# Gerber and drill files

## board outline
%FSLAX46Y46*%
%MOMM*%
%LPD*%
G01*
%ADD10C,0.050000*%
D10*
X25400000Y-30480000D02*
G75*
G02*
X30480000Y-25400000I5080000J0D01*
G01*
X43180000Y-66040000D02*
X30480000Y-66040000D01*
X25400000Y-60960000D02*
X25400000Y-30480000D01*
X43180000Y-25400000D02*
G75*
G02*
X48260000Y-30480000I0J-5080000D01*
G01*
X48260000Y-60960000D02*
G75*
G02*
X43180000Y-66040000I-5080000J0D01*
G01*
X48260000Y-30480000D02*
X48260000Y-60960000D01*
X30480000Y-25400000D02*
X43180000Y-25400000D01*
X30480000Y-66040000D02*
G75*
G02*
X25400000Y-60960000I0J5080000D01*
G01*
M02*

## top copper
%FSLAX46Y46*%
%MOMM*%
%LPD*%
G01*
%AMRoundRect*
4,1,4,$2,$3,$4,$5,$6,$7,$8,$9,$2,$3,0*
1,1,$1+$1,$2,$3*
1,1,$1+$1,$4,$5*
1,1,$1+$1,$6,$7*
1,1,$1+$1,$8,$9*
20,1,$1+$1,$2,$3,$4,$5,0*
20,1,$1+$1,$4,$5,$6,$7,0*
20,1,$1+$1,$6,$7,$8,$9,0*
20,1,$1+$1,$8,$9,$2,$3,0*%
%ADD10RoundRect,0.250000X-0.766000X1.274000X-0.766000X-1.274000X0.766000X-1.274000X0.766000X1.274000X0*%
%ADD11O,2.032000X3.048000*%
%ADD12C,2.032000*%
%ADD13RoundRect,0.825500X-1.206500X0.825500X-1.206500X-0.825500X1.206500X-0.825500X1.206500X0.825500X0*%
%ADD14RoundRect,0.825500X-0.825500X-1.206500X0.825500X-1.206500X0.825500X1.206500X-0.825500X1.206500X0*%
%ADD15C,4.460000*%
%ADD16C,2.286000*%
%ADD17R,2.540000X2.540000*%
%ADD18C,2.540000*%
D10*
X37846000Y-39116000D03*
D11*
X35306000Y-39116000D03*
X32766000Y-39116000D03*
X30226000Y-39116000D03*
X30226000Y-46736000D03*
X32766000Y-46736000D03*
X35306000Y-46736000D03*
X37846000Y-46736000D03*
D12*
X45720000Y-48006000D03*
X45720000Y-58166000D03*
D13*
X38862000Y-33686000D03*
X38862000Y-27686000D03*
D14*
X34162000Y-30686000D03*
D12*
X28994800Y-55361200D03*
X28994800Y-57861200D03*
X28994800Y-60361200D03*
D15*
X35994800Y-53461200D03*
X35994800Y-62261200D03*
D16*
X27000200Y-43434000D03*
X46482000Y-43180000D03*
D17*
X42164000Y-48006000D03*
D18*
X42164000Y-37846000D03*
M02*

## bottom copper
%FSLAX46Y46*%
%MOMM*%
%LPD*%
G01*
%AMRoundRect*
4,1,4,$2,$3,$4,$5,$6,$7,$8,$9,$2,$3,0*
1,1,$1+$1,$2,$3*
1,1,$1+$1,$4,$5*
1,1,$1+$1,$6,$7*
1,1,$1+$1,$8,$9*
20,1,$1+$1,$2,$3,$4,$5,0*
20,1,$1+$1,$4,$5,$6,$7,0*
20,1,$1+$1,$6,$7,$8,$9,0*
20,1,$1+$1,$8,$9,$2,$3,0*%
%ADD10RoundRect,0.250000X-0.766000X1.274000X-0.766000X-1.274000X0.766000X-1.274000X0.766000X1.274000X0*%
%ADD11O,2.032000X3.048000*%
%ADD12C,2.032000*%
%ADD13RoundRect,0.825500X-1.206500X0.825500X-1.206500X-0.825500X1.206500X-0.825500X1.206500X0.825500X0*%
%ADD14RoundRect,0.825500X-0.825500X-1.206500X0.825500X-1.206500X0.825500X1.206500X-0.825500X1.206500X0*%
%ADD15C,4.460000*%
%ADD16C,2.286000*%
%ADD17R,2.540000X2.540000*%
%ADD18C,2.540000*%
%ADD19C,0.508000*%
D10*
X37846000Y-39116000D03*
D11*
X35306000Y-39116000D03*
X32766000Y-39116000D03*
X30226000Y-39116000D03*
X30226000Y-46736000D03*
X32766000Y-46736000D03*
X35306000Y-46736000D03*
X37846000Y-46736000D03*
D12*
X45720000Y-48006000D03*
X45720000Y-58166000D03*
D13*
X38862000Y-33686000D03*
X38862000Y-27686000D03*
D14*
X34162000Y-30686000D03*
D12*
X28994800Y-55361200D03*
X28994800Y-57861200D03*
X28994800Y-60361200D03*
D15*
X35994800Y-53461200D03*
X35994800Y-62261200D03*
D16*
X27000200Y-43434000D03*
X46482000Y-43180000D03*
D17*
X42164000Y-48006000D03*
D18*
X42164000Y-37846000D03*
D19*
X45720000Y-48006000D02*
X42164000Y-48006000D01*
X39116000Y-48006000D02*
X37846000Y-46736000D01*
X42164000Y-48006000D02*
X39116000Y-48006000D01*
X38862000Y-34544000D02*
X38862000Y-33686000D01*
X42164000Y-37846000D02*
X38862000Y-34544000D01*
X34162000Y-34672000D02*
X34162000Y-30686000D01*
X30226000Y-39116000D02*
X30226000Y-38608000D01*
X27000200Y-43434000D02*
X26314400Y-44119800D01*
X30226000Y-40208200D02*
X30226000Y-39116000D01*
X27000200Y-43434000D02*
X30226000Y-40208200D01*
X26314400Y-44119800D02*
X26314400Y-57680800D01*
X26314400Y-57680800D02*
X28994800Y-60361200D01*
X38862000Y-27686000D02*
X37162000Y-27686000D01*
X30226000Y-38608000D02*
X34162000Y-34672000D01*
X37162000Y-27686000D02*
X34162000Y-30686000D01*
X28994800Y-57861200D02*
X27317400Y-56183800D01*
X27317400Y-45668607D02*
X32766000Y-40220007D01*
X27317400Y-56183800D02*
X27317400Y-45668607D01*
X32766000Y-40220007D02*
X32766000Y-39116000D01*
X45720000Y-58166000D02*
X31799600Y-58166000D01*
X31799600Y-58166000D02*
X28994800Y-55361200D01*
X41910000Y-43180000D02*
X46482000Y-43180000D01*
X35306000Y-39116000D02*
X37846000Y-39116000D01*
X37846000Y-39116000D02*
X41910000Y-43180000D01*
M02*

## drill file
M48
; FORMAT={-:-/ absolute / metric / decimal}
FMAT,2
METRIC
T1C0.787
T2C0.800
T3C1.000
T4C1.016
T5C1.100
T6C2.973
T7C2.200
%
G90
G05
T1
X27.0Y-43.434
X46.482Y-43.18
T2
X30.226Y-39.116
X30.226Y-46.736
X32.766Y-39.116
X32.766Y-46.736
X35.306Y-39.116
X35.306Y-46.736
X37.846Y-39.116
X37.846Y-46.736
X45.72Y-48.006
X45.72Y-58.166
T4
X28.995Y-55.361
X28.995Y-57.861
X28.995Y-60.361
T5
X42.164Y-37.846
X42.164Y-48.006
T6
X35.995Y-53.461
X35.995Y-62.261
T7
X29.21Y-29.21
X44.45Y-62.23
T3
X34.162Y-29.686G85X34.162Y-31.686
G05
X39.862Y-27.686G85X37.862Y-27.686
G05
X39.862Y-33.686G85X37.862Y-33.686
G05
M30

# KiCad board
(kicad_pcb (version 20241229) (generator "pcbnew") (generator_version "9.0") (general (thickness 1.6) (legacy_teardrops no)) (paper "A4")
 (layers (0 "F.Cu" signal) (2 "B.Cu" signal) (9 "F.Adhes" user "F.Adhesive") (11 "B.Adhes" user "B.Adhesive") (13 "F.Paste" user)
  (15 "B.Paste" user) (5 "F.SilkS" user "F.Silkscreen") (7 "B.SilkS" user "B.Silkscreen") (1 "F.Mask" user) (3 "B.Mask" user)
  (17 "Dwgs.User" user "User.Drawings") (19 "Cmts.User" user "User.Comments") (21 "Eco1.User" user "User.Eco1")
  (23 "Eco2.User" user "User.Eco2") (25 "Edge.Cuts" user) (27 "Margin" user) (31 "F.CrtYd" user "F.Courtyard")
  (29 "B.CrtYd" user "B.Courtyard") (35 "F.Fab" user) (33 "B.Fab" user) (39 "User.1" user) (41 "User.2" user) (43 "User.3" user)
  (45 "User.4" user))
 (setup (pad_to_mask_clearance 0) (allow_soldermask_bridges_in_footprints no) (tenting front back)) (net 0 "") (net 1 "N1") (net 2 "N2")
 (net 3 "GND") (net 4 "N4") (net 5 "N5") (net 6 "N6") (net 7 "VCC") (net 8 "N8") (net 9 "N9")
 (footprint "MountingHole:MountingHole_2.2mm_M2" (layer "F.Cu") (at 29.21 29.21)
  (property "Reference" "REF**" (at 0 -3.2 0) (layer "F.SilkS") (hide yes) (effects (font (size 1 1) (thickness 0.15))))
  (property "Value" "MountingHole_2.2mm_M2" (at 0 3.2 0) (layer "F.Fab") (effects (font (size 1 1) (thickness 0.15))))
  (pad "" np_thru_hole circle (at 0 0) (size 2.2 2.2) (drill 2.2) (layers "*.Cu" "*.Mask")))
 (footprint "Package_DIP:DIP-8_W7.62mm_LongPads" (layer "F.Cu") (at 37.846 39.116 -90)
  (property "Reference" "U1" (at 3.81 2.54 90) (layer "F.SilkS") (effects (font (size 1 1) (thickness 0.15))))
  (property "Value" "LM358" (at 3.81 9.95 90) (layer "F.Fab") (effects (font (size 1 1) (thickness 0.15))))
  (pad "1" thru_hole roundrect (at 0 0 270) (size 3.048 2.032) (drill 0.8) (layers "*.Cu" "*.Mask") (remove_unused_layers no)
   (roundrect_rratio 0.1230314961) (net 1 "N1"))
  (pad "2" thru_hole oval (at 0 2.54 270) (size 3.048 2.032) (drill 0.8) (layers "*.Cu" "*.Mask") (remove_unused_layers no) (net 1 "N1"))
  (pad "3" thru_hole oval (at 0 5.08 270) (size 3.048 2.032) (drill 0.8) (layers "*.Cu" "*.Mask") (remove_unused_layers no) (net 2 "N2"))
  (pad "4" thru_hole oval (at 0 7.62 270) (size 3.048 2.032) (drill 0.8) (layers "*.Cu" "*.Mask") (remove_unused_layers no) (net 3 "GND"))
  (pad "5" thru_hole oval (at 7.62 7.62 270) (size 3.048 2.032) (drill 0.8) (layers "*.Cu" "*.Mask") (remove_unused_layers no) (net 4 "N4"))
  (pad "6" thru_hole oval (at 7.62 5.08 270) (size 3.048 2.032) (drill 0.8) (layers "*.Cu" "*.Mask") (remove_unused_layers no) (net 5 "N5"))
  (pad "7" thru_hole oval (at 7.62 2.54 270) (size 3.048 2.032) (drill 0.8) (layers "*.Cu" "*.Mask") (remove_unused_layers no) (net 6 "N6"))
  (pad "8" thru_hole oval (at 7.62 0 270) (size 3.048 2.032) (drill 0.8) (layers "*.Cu" "*.Mask") (remove_unused_layers no) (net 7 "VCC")))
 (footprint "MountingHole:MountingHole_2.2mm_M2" (layer "F.Cu") (at 44.45 62.23)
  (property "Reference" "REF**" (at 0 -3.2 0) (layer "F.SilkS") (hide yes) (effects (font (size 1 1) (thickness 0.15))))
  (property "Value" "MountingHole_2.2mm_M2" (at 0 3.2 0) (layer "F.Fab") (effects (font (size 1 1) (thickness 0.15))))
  (pad "" np_thru_hole circle (at 0 0) (size 2.2 2.2) (drill 2.2) (layers "*.Cu" "*.Mask")))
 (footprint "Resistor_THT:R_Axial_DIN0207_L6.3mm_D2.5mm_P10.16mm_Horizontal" (layer "F.Cu") (at 45.72 48.006 -90)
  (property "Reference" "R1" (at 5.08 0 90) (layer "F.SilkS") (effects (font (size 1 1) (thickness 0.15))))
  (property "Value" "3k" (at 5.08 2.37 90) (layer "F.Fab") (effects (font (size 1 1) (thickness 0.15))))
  (pad "1" thru_hole circle (at 0 0 270) (size 2.032 2.032) (drill 0.8) (layers "*.Cu" "*.Mask") (remove_unused_layers no) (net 7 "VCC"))
  (pad "2" thru_hole circle (at 10.16 0 270) (size 2.032 2.032) (drill 0.8) (layers "*.Cu" "*.Mask") (remove_unused_layers no) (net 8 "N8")))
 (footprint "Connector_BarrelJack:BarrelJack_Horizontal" (layer "F.Cu") (at 38.862 33.686 -90)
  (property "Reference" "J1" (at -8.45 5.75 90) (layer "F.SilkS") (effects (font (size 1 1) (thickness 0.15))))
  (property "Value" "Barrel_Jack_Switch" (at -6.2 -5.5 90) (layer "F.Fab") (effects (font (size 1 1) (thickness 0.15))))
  (pad "1" thru_hole roundrect (at 0 0 270) (size 3.302 4.064) (drill oval 1 3) (layers "*.Cu" "*.Mask") (remove_unused_layers no)
   (roundrect_rratio 0.25) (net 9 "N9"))
  (pad "2" thru_hole roundrect (at -6 0 270) (size 3.302 4.064) (drill oval 1 3) (layers "*.Cu" "*.Mask") (remove_unused_layers no)
   (roundrect_rratio 0.25) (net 3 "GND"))
  (pad "3" thru_hole roundrect (at -3 4.7) (size 3.302 4.064) (drill oval 1 3) (layers "*.Cu" "*.Mask") (remove_unused_layers no)
   (roundrect_rratio 0.25) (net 3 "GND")))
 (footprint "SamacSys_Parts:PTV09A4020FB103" (layer "F.Cu") (at 34.5948 57.8612 -90)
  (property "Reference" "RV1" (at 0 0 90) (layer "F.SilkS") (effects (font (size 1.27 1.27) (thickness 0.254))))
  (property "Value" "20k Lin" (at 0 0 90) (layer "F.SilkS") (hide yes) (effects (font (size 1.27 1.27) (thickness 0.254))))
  (pad "1" thru_hole circle (at -2.5 5.6 270) (size 2.032 2.032) (drill 1.016) (layers "*.Cu" "*.Mask") (remove_unused_layers no)
   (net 8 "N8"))
  (pad "2" thru_hole circle (at 0 5.6 270) (size 2.032 2.032) (drill 1.016) (layers "*.Cu" "*.Mask") (remove_unused_layers no) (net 2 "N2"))
  (pad "3" thru_hole circle (at 2.5 5.6 270) (size 2.032 2.032) (drill 1.016) (layers "*.Cu" "*.Mask") (remove_unused_layers no)
   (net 3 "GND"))
  (pad "4" thru_hole circle (at -4.4 -1.4 270) (size 4.46 4.46) (drill 2.9732) (layers "*.Cu" "*.Mask") (remove_unused_layers no))
  (pad "5" thru_hole circle (at 4.4 -1.4 270) (size 4.46 4.46) (drill 2.9732) (layers "*.Cu" "*.Mask") (remove_unused_layers no)))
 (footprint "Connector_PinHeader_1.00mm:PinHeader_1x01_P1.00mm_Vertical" (layer "F.Cu") (at 27.0002 43.434)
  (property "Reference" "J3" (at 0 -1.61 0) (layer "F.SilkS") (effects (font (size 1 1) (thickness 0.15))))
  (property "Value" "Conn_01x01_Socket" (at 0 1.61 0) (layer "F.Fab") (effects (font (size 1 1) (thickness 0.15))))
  (pad "1" thru_hole circle (at 0 0) (size 2.286 2.286) (drill 0.7874) (layers "*.Cu" "*.Mask") (remove_unused_layers no) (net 3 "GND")))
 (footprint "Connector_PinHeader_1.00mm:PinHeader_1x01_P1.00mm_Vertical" (layer "F.Cu") (at 46.482 43.18)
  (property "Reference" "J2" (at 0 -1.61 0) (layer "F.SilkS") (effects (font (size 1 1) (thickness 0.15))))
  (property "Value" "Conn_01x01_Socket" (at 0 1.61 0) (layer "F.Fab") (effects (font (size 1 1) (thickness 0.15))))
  (pad "1" thru_hole circle (at 0 0) (size 2.286 2.286) (drill 0.7874) (layers "*.Cu" "*.Mask") (remove_unused_layers no) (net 1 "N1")))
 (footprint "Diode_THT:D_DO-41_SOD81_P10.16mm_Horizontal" (layer "F.Cu") (at 42.164 48.006 90)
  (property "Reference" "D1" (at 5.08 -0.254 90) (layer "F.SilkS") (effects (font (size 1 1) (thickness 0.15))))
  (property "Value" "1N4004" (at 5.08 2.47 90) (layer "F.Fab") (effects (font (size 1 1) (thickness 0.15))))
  (pad "1" thru_hole rect (at 0 0 90) (size 2.54 2.54) (drill 1.1) (layers "*.Cu" "*.Mask") (remove_unused_layers no) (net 7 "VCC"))
  (pad "2" thru_hole circle (at 10.16 0 90) (size 2.54 2.54) (drill 1.1) (layers "*.Cu" "*.Mask") (remove_unused_layers no) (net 9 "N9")))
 (gr_arc (start 25.4 30.48) (mid 26.887898 26.887898) (end 30.48 25.4) (stroke (width 0.05) (type default)) (layer "Edge.Cuts"))
 (gr_line (start 43.18 66.04) (end 30.48 66.04) (stroke (width 0.05) (type default)) (layer "Edge.Cuts"))
 (gr_line (start 25.4 60.96) (end 25.4 30.48) (stroke (width 0.05) (type default)) (layer "Edge.Cuts"))
 (gr_arc (start 43.18 25.4) (mid 46.772102 26.887898) (end 48.26 30.48) (stroke (width 0.05) (type default)) (layer "Edge.Cuts"))
 (gr_arc (start 48.26 60.96) (mid 46.772102 64.552102) (end 43.18 66.04) (stroke (width 0.05) (type default)) (layer "Edge.Cuts"))
 (gr_line (start 48.26 30.48) (end 48.26 60.96) (stroke (width 0.05) (type default)) (layer "Edge.Cuts"))
 (gr_line (start 30.48 25.4) (end 43.18 25.4) (stroke (width 0.05) (type default)) (layer "Edge.Cuts"))
 (gr_arc (start 30.48 66.04) (mid 26.887898 64.552102) (end 25.4 60.96) (stroke (width 0.05) (type default)) (layer "Edge.Cuts"))
 (segment (start 45.72 48.006) (end 42.164 48.006) (width 0.508) (layer "B.Cu") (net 7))
 (segment (start 39.116 48.006) (end 37.846 46.736) (width 0.508) (layer "B.Cu") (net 7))
 (segment (start 42.164 48.006) (end 39.116 48.006) (width 0.508) (layer "B.Cu") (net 7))
 (segment (start 38.862 34.544) (end 38.862 33.686) (width 0.508) (layer "B.Cu") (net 9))
 (segment (start 42.164 37.846) (end 38.862 34.544) (width 0.508) (layer "B.Cu") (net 9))
 (segment (start 34.162 34.672) (end 34.162 30.686) (width 0.508) (layer "B.Cu") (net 3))
 (segment (start 30.226 39.116) (end 30.226 38.608) (width 0.508) (layer "B.Cu") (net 3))
 (segment (start 27.0002 43.434) (end 26.3144 44.1198) (width 0.508) (layer "B.Cu") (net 3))
 (segment (start 30.226 40.2082) (end 30.226 39.116) (width 0.508) (layer "B.Cu") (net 3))
 (segment (start 27.0002 43.434) (end 30.226 40.2082) (width 0.508) (layer "B.Cu") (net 3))
 (segment (start 26.3144 44.1198) (end 26.3144 57.6808) (width 0.508) (layer "B.Cu") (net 3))
 (segment (start 26.3144 57.6808) (end 28.9948 60.3612) (width 0.508) (layer "B.Cu") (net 3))
 (segment (start 38.862 27.686) (end 37.162 27.686) (width 0.508) (layer "B.Cu") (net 3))
 (segment (start 30.226 38.608) (end 34.162 34.672) (width 0.508) (layer "B.Cu") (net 3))
 (segment (start 37.162 27.686) (end 34.162 30.686) (width 0.508) (layer "B.Cu") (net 3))
 (segment (start 28.9948 57.8612) (end 27.3174 56.1838) (width 0.508) (layer "B.Cu") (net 2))
 (segment (start 27.3174 45.668607) (end 32.766 40.220007) (width 0.508) (layer "B.Cu") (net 2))
 (segment (start 27.3174 56.1838) (end 27.3174 45.668607) (width 0.508) (layer "B.Cu") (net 2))
 (segment (start 32.766 40.220007) (end 32.766 39.116) (width 0.508) (layer "B.Cu") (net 2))
 (segment (start 45.72 58.166) (end 31.7996 58.166) (width 0.508) (layer "B.Cu") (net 8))
 (segment (start 31.7996 58.166) (end 28.9948 55.3612) (width 0.508) (layer "B.Cu") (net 8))
 (segment (start 41.91 43.18) (end 46.482 43.18) (width 0.508) (layer "B.Cu") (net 1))
 (segment (start 35.306 39.116) (end 37.846 39.116) (width 0.508) (layer "B.Cu") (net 1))
 (segment (start 37.846 39.116) (end 41.91 43.18) (width 0.508) (layer "B.Cu") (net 1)))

